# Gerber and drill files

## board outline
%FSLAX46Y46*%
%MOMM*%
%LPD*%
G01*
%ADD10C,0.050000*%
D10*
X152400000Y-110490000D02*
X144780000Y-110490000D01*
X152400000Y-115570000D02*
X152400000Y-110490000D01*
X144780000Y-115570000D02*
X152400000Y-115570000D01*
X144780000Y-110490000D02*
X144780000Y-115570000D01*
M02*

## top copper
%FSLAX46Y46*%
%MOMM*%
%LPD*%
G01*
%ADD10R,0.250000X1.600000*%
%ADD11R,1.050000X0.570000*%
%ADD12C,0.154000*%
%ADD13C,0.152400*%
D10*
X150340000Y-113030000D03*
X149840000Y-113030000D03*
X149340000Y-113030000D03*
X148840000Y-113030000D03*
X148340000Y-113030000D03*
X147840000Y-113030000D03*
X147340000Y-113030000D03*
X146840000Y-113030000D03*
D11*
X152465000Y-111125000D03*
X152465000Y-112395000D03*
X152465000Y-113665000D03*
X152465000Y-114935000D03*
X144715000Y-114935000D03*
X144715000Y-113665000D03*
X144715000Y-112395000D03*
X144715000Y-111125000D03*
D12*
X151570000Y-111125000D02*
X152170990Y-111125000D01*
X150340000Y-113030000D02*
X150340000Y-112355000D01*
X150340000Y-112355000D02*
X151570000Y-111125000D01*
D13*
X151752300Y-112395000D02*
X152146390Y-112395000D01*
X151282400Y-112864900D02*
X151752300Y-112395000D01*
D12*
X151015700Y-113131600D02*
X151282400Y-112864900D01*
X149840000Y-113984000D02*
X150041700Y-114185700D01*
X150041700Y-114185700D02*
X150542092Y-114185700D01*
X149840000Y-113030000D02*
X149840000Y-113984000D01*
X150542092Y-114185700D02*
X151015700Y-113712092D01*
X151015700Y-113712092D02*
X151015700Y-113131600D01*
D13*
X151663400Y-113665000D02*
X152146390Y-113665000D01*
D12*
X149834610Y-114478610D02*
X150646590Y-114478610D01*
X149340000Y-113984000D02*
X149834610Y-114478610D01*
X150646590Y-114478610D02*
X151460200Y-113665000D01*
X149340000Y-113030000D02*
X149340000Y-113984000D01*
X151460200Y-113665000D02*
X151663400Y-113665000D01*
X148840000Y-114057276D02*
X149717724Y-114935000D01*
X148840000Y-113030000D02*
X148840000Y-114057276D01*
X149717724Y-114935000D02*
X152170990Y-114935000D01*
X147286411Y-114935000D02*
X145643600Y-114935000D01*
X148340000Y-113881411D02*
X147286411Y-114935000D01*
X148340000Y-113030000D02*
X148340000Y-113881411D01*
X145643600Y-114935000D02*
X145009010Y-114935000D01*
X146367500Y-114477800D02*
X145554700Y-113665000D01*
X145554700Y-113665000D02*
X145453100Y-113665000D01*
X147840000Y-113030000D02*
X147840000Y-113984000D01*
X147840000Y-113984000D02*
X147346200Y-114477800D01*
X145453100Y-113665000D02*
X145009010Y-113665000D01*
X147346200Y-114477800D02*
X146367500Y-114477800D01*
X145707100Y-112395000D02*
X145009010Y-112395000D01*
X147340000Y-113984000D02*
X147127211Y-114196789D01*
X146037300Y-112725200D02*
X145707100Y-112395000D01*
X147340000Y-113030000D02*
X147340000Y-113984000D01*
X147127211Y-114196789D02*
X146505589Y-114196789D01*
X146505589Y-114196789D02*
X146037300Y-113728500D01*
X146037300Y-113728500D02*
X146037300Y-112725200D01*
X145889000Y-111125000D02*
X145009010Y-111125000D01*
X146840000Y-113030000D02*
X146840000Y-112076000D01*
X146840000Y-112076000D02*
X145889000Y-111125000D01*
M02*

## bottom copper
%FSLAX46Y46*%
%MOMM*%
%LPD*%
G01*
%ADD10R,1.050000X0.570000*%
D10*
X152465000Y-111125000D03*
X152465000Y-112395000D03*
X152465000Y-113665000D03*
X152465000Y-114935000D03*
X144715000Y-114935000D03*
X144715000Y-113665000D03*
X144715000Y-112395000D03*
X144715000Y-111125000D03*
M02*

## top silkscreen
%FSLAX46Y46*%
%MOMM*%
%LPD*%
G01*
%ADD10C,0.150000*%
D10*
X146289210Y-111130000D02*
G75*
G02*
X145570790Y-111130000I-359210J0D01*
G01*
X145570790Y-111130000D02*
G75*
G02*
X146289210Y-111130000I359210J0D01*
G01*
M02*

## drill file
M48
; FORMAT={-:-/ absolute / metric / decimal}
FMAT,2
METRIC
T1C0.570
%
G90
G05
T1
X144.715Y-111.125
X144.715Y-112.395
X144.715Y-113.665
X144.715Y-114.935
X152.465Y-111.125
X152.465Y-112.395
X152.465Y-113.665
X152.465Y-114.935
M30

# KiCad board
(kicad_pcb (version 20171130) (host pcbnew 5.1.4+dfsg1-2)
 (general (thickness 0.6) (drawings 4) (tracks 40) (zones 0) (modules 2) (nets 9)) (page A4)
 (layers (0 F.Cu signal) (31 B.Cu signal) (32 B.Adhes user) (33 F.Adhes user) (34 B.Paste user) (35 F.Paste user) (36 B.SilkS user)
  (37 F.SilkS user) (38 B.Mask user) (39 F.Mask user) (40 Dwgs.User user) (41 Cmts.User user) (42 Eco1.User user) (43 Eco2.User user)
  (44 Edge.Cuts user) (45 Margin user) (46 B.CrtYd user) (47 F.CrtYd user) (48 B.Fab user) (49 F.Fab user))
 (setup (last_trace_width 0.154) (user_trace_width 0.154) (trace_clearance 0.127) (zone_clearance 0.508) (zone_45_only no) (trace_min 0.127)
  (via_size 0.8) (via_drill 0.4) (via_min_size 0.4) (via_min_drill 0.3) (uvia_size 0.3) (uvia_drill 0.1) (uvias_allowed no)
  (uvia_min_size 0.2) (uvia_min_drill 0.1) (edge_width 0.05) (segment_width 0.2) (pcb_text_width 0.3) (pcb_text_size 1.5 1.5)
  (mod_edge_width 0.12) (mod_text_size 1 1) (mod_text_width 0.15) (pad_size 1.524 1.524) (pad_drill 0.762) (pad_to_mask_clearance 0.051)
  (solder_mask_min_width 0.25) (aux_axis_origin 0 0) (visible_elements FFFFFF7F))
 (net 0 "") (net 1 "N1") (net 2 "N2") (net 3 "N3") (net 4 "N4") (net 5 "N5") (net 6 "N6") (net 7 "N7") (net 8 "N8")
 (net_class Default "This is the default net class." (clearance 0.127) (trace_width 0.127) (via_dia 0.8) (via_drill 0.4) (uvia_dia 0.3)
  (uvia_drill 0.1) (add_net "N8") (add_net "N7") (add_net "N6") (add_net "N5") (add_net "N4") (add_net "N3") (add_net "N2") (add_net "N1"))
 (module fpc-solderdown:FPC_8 (layer F.Cu) (at 148.59 113.03)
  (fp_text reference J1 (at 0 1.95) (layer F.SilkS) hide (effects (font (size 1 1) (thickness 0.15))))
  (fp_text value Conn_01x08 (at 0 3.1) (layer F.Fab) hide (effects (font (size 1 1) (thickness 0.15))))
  (pad 8 smd rect (at 1.75 0) (size 0.25 1.6) (layers F.Cu F.Paste F.Mask) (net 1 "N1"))
  (pad 7 smd rect (at 1.25 0) (size 0.25 1.6) (layers F.Cu F.Paste F.Mask) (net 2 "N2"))
  (pad 6 smd rect (at 0.75 0) (size 0.25 1.6) (layers F.Cu F.Paste F.Mask) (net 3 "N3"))
  (pad 5 smd rect (at 0.25 0) (size 0.25 1.6) (layers F.Cu F.Paste F.Mask) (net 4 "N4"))
  (pad 4 smd rect (at -0.25 0) (size 0.25 1.6) (layers F.Cu F.Paste F.Mask) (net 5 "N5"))
  (pad 3 smd rect (at -0.75 0) (size 0.25 1.6) (layers F.Cu F.Paste F.Mask) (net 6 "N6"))
  (pad 2 smd rect (at -1.25 0) (size 0.25 1.6) (layers F.Cu F.Paste F.Mask) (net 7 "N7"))
  (pad 1 smd rect (at -1.75 0) (size 0.25 1.6) (layers F.Cu F.Paste F.Mask) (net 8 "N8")))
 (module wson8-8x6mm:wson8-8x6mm (layer F.Cu) (at 148.59 113.03)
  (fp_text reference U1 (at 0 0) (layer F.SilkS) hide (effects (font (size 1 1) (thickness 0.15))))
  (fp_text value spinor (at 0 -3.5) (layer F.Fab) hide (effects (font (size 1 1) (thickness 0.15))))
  (fp_circle (center -2.66 -1.9) (end -2.30079 -1.9) (layer F.SilkS) (width 0.15))
  (pad 8 thru_hole rect (at 3.875 -1.905) (size 1.05 0.57) (drill 0.57) (layers *.Cu *.Mask) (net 1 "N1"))
  (pad 7 thru_hole rect (at 3.875 -0.635) (size 1.05 0.57) (drill 0.57) (layers *.Cu *.Mask) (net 2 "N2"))
  (pad 6 thru_hole rect (at 3.875 0.635) (size 1.05 0.57) (drill 0.57) (layers *.Cu *.Mask) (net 3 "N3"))
  (pad 5 thru_hole rect (at 3.875 1.905) (size 1.05 0.57) (drill 0.57) (layers *.Cu *.Mask) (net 4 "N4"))
  (pad 4 thru_hole rect (at -3.875 1.905) (size 1.05 0.57) (drill 0.57) (layers *.Cu *.Mask) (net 5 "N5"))
  (pad 3 thru_hole rect (at -3.875 0.635) (size 1.05 0.57) (drill 0.57) (layers *.Cu *.Mask) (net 6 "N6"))
  (pad 2 thru_hole rect (at -3.875 -0.635) (size 1.05 0.57) (drill 0.57) (layers *.Cu *.Mask) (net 7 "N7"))
  (pad 1 thru_hole rect (at -3.875 -1.905) (size 1.05 0.57) (drill 0.57) (layers *.Cu *.Mask) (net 8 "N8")))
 (gr_line (start 152.4 110.49) (end 144.78 110.49) (layer Edge.Cuts) (width 0.05))
 (gr_line (start 152.4 115.57) (end 152.4 110.49) (layer Edge.Cuts) (width 0.05))
 (gr_line (start 144.78 115.57) (end 152.4 115.57) (layer Edge.Cuts) (width 0.05))
 (gr_line (start 144.78 110.49) (end 144.78 115.57) (layer Edge.Cuts) (width 0.05))
 (segment (start 151.57 111.125) (end 152.17099 111.125) (width 0.154) (layer F.Cu) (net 1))
 (segment (start 150.34 113.03) (end 150.34 112.355) (width 0.154) (layer F.Cu) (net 1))
 (segment (start 150.34 112.355) (end 151.57 111.125) (width 0.154) (layer F.Cu) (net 1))
 (segment (start 151.7523 112.395) (end 152.14639 112.395) (width 0.1524) (layer F.Cu) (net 2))
 (segment (start 151.2824 112.8649) (end 151.7523 112.395) (width 0.1524) (layer F.Cu) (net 2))
 (segment (start 151.0157 113.1316) (end 151.2824 112.8649) (width 0.154) (layer F.Cu) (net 2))
 (segment (start 149.84 113.984) (end 150.0417 114.1857) (width 0.154) (layer F.Cu) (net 2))
 (segment (start 150.0417 114.1857) (end 150.542092 114.1857) (width 0.154) (layer F.Cu) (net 2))
 (segment (start 149.84 113.03) (end 149.84 113.984) (width 0.154) (layer F.Cu) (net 2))
 (segment (start 150.542092 114.1857) (end 151.0157 113.712092) (width 0.154) (layer F.Cu) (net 2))
 (segment (start 151.0157 113.712092) (end 151.0157 113.1316) (width 0.154) (layer F.Cu) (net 2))
 (segment (start 151.6634 113.665) (end 152.14639 113.665) (width 0.1524) (layer F.Cu) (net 3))
 (segment (start 149.83461 114.47861) (end 150.64659 114.47861) (width 0.154) (layer F.Cu) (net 3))
 (segment (start 149.34 113.984) (end 149.83461 114.47861) (width 0.154) (layer F.Cu) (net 3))
 (segment (start 150.64659 114.47861) (end 151.4602 113.665) (width 0.154) (layer F.Cu) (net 3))
 (segment (start 149.34 113.03) (end 149.34 113.984) (width 0.154) (layer F.Cu) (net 3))
 (segment (start 151.4602 113.665) (end 151.6634 113.665) (width 0.154) (layer F.Cu) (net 3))
 (segment (start 148.84 114.057276) (end 149.717724 114.935) (width 0.154) (layer F.Cu) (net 4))
 (segment (start 148.84 113.03) (end 148.84 114.057276) (width 0.154) (layer F.Cu) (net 4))
 (segment (start 149.717724 114.935) (end 152.17099 114.935) (width 0.154) (layer F.Cu) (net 4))
 (segment (start 147.286411 114.935) (end 145.6436 114.935) (width 0.154) (layer F.Cu) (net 5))
 (segment (start 148.34 113.881411) (end 147.286411 114.935) (width 0.154) (layer F.Cu) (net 5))
 (segment (start 148.34 113.03) (end 148.34 113.881411) (width 0.154) (layer F.Cu) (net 5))
 (segment (start 145.6436 114.935) (end 145.00901 114.935) (width 0.154) (layer F.Cu) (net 5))
 (segment (start 146.3675 114.4778) (end 145.5547 113.665) (width 0.154) (layer F.Cu) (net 6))
 (segment (start 145.5547 113.665) (end 145.4531 113.665) (width 0.154) (layer F.Cu) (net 6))
 (segment (start 147.84 113.03) (end 147.84 113.984) (width 0.154) (layer F.Cu) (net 6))
 (segment (start 147.84 113.984) (end 147.3462 114.4778) (width 0.154) (layer F.Cu) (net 6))
 (segment (start 145.4531 113.665) (end 145.00901 113.665) (width 0.154) (layer F.Cu) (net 6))
 (segment (start 147.3462 114.4778) (end 146.3675 114.4778) (width 0.154) (layer F.Cu) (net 6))
 (segment (start 145.7071 112.395) (end 145.00901 112.395) (width 0.154) (layer F.Cu) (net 7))
 (segment (start 147.34 113.984) (end 147.127211 114.196789) (width 0.154) (layer F.Cu) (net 7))
 (segment (start 146.0373 112.7252) (end 145.7071 112.395) (width 0.154) (layer F.Cu) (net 7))
 (segment (start 147.34 113.03) (end 147.34 113.984) (width 0.154) (layer F.Cu) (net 7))
 (segment (start 147.127211 114.196789) (end 146.505589 114.196789) (width 0.154) (layer F.Cu) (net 7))
 (segment (start 146.505589 114.196789) (end 146.0373 113.7285) (width 0.154) (layer F.Cu) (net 7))
 (segment (start 146.0373 113.7285) (end 146.0373 112.7252) (width 0.154) (layer F.Cu) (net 7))
 (segment (start 145.889 111.125) (end 145.00901 111.125) (width 0.154) (layer F.Cu) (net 8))
 (segment (start 146.84 113.03) (end 146.84 112.076) (width 0.154) (layer F.Cu) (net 8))
 (segment (start 146.84 112.076) (end 145.889 111.125) (width 0.154) (layer F.Cu) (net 8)))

